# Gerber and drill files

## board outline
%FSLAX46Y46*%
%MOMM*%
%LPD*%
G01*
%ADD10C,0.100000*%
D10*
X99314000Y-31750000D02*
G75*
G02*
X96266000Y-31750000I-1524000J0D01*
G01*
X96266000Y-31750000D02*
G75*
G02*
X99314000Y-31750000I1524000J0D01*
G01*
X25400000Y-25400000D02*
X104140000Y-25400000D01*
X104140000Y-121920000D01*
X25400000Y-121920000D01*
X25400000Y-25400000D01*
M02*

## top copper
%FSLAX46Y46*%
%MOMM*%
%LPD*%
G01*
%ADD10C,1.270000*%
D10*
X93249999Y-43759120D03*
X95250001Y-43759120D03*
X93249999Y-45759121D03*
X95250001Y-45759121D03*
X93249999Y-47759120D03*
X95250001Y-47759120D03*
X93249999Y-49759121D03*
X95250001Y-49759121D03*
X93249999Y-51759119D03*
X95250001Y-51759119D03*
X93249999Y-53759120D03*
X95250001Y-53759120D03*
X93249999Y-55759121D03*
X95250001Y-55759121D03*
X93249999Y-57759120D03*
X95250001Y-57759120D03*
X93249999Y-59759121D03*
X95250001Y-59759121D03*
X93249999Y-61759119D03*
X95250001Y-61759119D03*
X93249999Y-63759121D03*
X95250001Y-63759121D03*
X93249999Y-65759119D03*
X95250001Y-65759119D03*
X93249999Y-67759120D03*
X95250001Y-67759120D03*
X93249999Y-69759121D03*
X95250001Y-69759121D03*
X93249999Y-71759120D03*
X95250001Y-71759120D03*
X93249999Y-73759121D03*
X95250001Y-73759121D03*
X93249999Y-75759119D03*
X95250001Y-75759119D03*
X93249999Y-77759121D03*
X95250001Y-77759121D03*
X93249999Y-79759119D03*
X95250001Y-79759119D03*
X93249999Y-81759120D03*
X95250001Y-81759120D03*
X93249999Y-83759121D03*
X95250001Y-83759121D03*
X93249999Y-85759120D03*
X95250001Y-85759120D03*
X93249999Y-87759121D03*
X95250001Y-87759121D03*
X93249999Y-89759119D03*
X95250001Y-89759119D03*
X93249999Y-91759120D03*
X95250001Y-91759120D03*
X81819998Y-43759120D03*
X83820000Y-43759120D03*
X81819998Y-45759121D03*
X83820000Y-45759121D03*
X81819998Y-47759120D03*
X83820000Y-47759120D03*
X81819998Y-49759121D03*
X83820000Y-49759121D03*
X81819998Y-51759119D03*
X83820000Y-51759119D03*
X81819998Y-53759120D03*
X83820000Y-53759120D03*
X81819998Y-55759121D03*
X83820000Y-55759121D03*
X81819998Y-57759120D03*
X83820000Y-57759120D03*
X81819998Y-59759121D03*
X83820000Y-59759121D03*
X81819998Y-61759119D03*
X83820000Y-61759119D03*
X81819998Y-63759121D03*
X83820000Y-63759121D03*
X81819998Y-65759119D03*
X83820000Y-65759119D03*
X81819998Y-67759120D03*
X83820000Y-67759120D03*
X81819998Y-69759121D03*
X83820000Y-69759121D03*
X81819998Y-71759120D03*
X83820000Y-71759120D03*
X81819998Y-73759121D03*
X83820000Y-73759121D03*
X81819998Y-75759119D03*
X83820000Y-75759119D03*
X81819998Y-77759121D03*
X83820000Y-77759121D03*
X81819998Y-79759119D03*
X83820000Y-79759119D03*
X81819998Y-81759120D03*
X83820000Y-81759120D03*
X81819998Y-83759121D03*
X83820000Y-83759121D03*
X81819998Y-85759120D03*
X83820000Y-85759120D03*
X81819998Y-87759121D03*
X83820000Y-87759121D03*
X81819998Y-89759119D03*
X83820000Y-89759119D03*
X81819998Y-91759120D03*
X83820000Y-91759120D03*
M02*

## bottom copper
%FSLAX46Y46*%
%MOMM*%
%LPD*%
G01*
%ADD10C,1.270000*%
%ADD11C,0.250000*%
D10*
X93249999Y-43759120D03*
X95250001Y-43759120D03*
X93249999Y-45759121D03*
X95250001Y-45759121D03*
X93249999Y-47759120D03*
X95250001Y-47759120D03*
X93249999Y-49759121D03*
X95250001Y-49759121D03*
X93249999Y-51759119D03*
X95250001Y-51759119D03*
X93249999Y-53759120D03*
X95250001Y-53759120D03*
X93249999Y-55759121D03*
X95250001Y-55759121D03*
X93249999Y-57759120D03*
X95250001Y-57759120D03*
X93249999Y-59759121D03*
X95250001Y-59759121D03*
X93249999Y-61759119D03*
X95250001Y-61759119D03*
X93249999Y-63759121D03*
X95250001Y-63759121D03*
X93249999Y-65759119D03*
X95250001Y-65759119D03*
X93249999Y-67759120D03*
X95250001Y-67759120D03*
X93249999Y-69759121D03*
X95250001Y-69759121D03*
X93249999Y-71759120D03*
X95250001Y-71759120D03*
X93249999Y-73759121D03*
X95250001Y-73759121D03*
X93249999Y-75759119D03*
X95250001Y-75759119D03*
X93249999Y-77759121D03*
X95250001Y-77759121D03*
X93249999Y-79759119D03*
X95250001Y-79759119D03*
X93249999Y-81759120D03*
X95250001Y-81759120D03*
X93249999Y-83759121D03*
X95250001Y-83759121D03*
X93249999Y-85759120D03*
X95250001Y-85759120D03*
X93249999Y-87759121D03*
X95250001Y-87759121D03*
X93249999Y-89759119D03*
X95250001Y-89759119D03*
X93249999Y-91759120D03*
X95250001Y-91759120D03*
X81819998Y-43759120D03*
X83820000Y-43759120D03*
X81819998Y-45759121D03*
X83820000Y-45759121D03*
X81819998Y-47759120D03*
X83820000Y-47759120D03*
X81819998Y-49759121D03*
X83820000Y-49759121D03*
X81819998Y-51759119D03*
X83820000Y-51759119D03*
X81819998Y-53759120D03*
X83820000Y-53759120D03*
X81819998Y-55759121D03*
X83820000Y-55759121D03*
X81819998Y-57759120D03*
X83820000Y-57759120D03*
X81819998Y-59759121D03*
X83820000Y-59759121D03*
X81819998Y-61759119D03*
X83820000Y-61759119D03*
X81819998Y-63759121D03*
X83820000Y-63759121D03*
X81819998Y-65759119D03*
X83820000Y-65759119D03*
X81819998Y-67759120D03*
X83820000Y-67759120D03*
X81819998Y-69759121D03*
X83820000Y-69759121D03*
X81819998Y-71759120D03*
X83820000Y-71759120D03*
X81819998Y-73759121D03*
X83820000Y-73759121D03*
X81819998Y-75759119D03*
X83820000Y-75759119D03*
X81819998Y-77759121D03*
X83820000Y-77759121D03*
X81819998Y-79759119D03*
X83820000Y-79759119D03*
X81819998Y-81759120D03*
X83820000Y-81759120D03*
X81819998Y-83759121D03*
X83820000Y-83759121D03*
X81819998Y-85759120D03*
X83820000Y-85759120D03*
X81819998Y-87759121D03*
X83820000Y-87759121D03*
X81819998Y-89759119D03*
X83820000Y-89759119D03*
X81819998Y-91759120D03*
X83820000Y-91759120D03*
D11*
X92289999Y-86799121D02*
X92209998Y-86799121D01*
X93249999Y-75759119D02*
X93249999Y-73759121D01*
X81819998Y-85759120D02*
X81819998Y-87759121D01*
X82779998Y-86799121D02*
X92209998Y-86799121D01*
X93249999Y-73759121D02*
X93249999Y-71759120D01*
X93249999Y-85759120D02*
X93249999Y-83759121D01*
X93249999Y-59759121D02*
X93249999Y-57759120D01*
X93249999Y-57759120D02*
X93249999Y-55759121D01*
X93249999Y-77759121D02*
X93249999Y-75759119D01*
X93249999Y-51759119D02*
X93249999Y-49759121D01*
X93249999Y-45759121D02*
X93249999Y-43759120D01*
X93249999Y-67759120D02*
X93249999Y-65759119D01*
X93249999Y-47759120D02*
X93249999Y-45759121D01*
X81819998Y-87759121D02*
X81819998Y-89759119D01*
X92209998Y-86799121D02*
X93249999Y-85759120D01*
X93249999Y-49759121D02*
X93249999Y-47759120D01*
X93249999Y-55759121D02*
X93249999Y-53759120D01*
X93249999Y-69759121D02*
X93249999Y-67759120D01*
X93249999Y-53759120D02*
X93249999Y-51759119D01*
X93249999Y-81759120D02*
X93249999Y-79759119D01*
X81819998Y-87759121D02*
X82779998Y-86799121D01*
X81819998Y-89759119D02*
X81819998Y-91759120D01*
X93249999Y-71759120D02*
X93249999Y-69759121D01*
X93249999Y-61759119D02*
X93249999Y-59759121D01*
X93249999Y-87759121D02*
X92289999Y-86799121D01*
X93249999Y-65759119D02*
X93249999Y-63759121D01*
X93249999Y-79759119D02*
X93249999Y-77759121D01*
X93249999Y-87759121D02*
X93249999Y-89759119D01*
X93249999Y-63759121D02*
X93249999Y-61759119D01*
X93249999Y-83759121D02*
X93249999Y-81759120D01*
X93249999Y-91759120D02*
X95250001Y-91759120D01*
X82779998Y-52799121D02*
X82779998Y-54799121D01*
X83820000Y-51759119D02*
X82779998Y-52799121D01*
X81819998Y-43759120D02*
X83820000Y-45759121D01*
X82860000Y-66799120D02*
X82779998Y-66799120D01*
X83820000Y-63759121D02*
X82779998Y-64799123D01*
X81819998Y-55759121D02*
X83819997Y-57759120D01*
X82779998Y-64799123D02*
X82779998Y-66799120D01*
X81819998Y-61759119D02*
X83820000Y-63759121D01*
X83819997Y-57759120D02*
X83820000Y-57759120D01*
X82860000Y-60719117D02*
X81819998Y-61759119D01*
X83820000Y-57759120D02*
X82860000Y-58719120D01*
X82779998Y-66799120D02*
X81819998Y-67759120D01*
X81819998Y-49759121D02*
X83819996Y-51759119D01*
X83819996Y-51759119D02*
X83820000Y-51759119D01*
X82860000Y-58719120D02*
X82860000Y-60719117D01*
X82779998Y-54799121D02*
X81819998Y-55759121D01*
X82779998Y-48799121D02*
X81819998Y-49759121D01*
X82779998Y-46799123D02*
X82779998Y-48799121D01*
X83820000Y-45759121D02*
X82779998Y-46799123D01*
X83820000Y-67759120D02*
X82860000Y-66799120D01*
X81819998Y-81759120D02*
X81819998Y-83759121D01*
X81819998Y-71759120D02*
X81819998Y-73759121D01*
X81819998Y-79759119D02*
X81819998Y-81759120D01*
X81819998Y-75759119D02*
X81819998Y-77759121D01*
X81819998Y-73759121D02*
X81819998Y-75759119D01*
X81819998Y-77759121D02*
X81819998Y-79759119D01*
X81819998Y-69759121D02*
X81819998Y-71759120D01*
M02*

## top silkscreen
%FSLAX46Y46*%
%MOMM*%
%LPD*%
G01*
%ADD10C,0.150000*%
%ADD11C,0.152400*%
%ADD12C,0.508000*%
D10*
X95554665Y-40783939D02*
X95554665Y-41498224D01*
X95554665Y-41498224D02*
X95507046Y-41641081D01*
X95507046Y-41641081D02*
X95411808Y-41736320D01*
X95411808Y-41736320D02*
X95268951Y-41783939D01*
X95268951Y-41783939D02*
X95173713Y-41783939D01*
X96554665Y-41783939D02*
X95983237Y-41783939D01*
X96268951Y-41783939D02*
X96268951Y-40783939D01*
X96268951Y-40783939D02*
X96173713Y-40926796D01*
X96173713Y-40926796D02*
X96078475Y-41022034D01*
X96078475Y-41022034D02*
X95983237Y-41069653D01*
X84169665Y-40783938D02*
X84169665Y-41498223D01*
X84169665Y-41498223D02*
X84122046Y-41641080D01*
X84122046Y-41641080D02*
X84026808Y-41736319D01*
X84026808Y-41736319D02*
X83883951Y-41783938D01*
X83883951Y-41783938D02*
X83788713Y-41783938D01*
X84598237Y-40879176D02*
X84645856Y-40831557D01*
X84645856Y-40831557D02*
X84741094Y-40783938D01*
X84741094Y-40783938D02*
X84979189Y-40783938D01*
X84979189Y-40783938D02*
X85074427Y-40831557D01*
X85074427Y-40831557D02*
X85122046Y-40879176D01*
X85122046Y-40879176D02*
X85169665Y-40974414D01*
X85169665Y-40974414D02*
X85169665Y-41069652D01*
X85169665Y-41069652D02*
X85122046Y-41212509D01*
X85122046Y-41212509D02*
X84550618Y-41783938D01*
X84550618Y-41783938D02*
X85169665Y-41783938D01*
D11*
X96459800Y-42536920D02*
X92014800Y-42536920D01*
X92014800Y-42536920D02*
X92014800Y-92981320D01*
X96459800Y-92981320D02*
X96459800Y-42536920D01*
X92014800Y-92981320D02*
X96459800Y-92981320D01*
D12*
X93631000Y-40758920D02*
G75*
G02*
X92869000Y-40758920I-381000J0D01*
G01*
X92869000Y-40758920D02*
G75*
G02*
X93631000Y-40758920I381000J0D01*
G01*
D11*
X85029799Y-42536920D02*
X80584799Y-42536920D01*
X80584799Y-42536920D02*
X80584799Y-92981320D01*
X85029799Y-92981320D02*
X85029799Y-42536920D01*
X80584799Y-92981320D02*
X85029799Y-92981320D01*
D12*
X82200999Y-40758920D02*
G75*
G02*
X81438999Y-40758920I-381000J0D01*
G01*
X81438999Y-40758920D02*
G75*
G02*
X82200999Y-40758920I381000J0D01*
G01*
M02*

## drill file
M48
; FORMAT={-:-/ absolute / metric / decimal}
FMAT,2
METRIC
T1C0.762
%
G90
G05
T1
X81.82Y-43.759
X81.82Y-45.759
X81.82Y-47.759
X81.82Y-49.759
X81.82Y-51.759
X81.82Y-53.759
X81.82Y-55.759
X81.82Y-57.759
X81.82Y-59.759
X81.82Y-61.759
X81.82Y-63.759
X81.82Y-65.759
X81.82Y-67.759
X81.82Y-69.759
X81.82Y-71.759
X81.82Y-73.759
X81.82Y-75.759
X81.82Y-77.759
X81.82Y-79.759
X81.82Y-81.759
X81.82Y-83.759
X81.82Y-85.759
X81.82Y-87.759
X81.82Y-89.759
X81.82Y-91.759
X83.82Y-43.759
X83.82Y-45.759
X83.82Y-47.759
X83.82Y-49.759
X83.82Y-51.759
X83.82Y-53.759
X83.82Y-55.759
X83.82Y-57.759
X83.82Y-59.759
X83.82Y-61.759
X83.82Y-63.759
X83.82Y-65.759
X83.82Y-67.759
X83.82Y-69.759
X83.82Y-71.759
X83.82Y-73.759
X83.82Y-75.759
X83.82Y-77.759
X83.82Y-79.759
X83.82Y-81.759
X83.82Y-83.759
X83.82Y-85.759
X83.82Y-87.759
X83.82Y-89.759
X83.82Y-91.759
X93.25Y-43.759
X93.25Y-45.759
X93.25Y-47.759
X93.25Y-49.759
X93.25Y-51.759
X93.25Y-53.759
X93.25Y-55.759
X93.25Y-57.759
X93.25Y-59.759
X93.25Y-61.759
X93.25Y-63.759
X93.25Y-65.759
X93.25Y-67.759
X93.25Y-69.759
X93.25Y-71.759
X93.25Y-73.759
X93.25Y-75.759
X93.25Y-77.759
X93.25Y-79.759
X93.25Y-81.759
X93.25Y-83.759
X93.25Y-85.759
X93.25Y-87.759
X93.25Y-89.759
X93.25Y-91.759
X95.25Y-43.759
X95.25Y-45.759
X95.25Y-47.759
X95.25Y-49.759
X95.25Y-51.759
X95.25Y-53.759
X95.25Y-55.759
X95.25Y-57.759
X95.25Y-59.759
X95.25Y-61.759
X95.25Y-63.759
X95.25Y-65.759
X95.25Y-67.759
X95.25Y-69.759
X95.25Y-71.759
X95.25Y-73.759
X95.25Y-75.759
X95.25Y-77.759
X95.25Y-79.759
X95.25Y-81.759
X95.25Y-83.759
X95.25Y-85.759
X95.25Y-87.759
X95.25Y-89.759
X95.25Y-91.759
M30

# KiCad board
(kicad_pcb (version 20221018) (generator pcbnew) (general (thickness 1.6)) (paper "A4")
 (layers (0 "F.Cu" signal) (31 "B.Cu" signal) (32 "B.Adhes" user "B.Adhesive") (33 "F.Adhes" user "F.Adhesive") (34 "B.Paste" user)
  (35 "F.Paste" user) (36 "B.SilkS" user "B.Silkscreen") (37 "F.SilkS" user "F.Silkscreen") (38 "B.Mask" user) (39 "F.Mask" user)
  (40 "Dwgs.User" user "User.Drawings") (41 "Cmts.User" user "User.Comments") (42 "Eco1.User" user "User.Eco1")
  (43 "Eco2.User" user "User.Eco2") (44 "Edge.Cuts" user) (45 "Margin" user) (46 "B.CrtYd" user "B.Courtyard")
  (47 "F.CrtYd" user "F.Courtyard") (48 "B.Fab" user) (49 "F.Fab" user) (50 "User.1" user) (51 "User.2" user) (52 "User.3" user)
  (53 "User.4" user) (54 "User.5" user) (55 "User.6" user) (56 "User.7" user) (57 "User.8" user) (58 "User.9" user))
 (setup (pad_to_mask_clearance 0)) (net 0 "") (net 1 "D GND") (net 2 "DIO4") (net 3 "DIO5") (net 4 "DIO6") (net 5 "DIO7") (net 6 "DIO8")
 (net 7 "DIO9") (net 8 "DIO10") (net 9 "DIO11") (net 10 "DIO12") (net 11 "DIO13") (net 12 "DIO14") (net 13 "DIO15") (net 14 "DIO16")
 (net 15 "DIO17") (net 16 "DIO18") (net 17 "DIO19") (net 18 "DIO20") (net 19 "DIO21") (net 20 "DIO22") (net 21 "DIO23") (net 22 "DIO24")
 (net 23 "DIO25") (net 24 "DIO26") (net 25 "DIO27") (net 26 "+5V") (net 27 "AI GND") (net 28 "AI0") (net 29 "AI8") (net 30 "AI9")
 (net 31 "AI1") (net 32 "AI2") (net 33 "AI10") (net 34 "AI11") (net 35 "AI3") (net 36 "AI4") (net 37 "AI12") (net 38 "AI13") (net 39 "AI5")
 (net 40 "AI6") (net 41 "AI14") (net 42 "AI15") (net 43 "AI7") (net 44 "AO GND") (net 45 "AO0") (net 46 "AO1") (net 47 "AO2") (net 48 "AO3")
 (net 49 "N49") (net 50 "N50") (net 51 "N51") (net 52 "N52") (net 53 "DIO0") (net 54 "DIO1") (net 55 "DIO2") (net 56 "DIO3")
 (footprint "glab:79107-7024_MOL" (layer "F.Cu") (at 93.25 43.75912 -90)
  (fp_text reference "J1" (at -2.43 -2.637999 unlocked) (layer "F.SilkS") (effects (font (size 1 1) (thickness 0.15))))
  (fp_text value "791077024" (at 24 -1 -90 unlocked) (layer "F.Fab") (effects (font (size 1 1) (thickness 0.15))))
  (fp_line (start -1.2222 -3.2098) (end -1.2222 1.2352) (stroke (width 0.1524) (type solid)) (layer "F.SilkS"))
  (fp_line (start -1.2222 1.2352) (end 49.2222 1.2352) (stroke (width 0.1524) (type solid)) (layer "F.SilkS"))
  (fp_line (start 49.2222 -3.2098) (end -1.2222 -3.2098) (stroke (width 0.1524) (type solid)) (layer "F.SilkS"))
  (fp_line (start 49.2222 1.2352) (end 49.2222 -3.2098) (stroke (width 0.1524) (type solid)) (layer "F.SilkS"))
  (fp_circle (center -3.0002 0) (end -2.6192 0) (stroke (width 0.508) (type solid)) (fill none) (layer "F.SilkS"))
  (pad "1" thru_hole circle (at 0 0.000001 270) (size 1.27 1.27) (drill 0.762) (layers "*.Cu" "*.Mask") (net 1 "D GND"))
  (pad "2" thru_hole circle (at 0 -2.000001 270) (size 1.27 1.27) (drill 0.762) (layers "*.Cu" "*.Mask") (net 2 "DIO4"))
  (pad "3" thru_hole circle (at 2.000001 0.000001 270) (size 1.27 1.27) (drill 0.762) (layers "*.Cu" "*.Mask") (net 1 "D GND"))
  (pad "4" thru_hole circle (at 2.000001 -2.000001 270) (size 1.27 1.27) (drill 0.762) (layers "*.Cu" "*.Mask") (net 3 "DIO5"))
  (pad "5" thru_hole circle (at 4 0.000001 270) (size 1.27 1.27) (drill 0.762) (layers "*.Cu" "*.Mask") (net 1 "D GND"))
  (pad "6" thru_hole circle (at 4 -2.000001 270) (size 1.27 1.27) (drill 0.762) (layers "*.Cu" "*.Mask") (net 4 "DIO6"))
  (pad "7" thru_hole circle (at 6.000001 0.000001 270) (size 1.27 1.27) (drill 0.762) (layers "*.Cu" "*.Mask") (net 1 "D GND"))
  (pad "8" thru_hole circle (at 6.000001 -2.000001 270) (size 1.27 1.27) (drill 0.762) (layers "*.Cu" "*.Mask") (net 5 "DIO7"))
  (pad "9" thru_hole circle (at 7.999999 0.000001 270) (size 1.27 1.27) (drill 0.762) (layers "*.Cu" "*.Mask") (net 1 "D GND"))
  (pad "10" thru_hole circle (at 7.999999 -2.000001 270) (size 1.27 1.27) (drill 0.762) (layers "*.Cu" "*.Mask") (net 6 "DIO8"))
  (pad "11" thru_hole circle (at 10 0.000001 270) (size 1.27 1.27) (drill 0.762) (layers "*.Cu" "*.Mask") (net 1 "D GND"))
  (pad "12" thru_hole circle (at 10 -2.000001 270) (size 1.27 1.27) (drill 0.762) (layers "*.Cu" "*.Mask") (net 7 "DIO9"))
  (pad "13" thru_hole circle (at 12.000001 0.000001 270) (size 1.27 1.27) (drill 0.762) (layers "*.Cu" "*.Mask") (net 1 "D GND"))
  (pad "14" thru_hole circle (at 12.000001 -2.000001 270) (size 1.27 1.27) (drill 0.762) (layers "*.Cu" "*.Mask") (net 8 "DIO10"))
  (pad "15" thru_hole circle (at 14 0.000001 270) (size 1.27 1.27) (drill 0.762) (layers "*.Cu" "*.Mask") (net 1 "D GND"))
  (pad "16" thru_hole circle (at 14 -2.000001 270) (size 1.27 1.27) (drill 0.762) (layers "*.Cu" "*.Mask") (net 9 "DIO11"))
  (pad "17" thru_hole circle (at 16.000001 0.000001 270) (size 1.27 1.27) (drill 0.762) (layers "*.Cu" "*.Mask") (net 1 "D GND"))
  (pad "18" thru_hole circle (at 16.000001 -2.000001 270) (size 1.27 1.27) (drill 0.762) (layers "*.Cu" "*.Mask") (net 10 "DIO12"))
  (pad "19" thru_hole circle (at 17.999999 0.000001 270) (size 1.27 1.27) (drill 0.762) (layers "*.Cu" "*.Mask") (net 1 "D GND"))
  (pad "20" thru_hole circle (at 17.999999 -2.000001 270) (size 1.27 1.27) (drill 0.762) (layers "*.Cu" "*.Mask") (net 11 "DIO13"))
  (pad "21" thru_hole circle (at 20.000001 0.000001 270) (size 1.27 1.27) (drill 0.762) (layers "*.Cu" "*.Mask") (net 1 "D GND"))
  (pad "22" thru_hole circle (at 20.000001 -2.000001 270) (size 1.27 1.27) (drill 0.762) (layers "*.Cu" "*.Mask") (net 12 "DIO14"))
  (pad "23" thru_hole circle (at 21.999999 0.000001 270) (size 1.27 1.27) (drill 0.762) (layers "*.Cu" "*.Mask") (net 1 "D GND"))
  (pad "24" thru_hole circle (at 21.999999 -2.000001 270) (size 1.27 1.27) (drill 0.762) (layers "*.Cu" "*.Mask") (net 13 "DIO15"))
  (pad "25" thru_hole circle (at 24 0.000001 270) (size 1.27 1.27) (drill 0.762) (layers "*.Cu" "*.Mask") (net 1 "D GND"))
  (pad "26" thru_hole circle (at 24 -2.000001 270) (size 1.27 1.27) (drill 0.762) (layers "*.Cu" "*.Mask") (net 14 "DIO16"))
  (pad "27" thru_hole circle (at 26.000001 0.000001 270) (size 1.27 1.27) (drill 0.762) (layers "*.Cu" "*.Mask") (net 1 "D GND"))
  (pad "28" thru_hole circle (at 26.000001 -2.000001 270) (size 1.27 1.27) (drill 0.762) (layers "*.Cu" "*.Mask") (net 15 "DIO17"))
  (pad "29" thru_hole circle (at 28 0.000001 270) (size 1.27 1.27) (drill 0.762) (layers "*.Cu" "*.Mask") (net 1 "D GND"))
  (pad "30" thru_hole circle (at 28 -2.000001 270) (size 1.27 1.27) (drill 0.762) (layers "*.Cu" "*.Mask") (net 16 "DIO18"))
  (pad "31" thru_hole circle (at 30.000001 0.000001 270) (size 1.27 1.27) (drill 0.762) (layers "*.Cu" "*.Mask") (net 1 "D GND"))
  (pad "32" thru_hole circle (at 30.000001 -2.000001 270) (size 1.27 1.27) (drill 0.762) (layers "*.Cu" "*.Mask") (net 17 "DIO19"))
  (pad "33" thru_hole circle (at 31.999999 0.000001 270) (size 1.27 1.27) (drill 0.762) (layers "*.Cu" "*.Mask") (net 1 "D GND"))
  (pad "34" thru_hole circle (at 31.999999 -2.000001 270) (size 1.27 1.27) (drill 0.762) (layers "*.Cu" "*.Mask") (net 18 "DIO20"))
  (pad "35" thru_hole circle (at 34.000001 0.000001 270) (size 1.27 1.27) (drill 0.762) (layers "*.Cu" "*.Mask") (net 1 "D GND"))
  (pad "36" thru_hole circle (at 34.000001 -2.000001 270) (size 1.27 1.27) (drill 0.762) (layers "*.Cu" "*.Mask") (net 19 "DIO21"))
  (pad "37" thru_hole circle (at 35.999999 0.000001 270) (size 1.27 1.27) (drill 0.762) (layers "*.Cu" "*.Mask") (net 1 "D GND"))
  (pad "38" thru_hole circle (at 35.999999 -2.000001 270) (size 1.27 1.27) (drill 0.762) (layers "*.Cu" "*.Mask") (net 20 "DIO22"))
  (pad "39" thru_hole circle (at 38 0.000001 270) (size 1.27 1.27) (drill 0.762) (layers "*.Cu" "*.Mask") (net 1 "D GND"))
  (pad "40" thru_hole circle (at 38 -2.000001 270) (size 1.27 1.27) (drill 0.762) (layers "*.Cu" "*.Mask") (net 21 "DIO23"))
  (pad "41" thru_hole circle (at 40.000001 0.000001 270) (size 1.27 1.27) (drill 0.762) (layers "*.Cu" "*.Mask") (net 1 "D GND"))
  (pad "42" thru_hole circle (at 40.000001 -2.000001 270) (size 1.27 1.27) (drill 0.762) (layers "*.Cu" "*.Mask") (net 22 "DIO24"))
  (pad "43" thru_hole circle (at 42 0.000001 270) (size 1.27 1.27) (drill 0.762) (layers "*.Cu" "*.Mask") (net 1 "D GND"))
  (pad "44" thru_hole circle (at 42 -2.000001 270) (size 1.27 1.27) (drill 0.762) (layers "*.Cu" "*.Mask") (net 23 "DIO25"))
  (pad "45" thru_hole circle (at 44.000001 0.000001 270) (size 1.27 1.27) (drill 0.762) (layers "*.Cu" "*.Mask") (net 1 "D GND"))
  (pad "46" thru_hole circle (at 44.000001 -2.000001 270) (size 1.27 1.27) (drill 0.762) (layers "*.Cu" "*.Mask") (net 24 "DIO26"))
  (pad "47" thru_hole circle (at 45.999999 0.000001 270) (size 1.27 1.27) (drill 0.762) (layers "*.Cu" "*.Mask") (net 1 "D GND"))
  (pad "48" thru_hole circle (at 45.999999 -2.000001 270) (size 1.27 1.27) (drill 0.762) (layers "*.Cu" "*.Mask") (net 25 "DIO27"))
  (pad "49" thru_hole circle (at 48 0.000001 270) (size 1.27 1.27) (drill 0.762) (layers "*.Cu" "*.Mask") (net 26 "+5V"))
  (pad "50" thru_hole circle (at 48 -2.000001 270) (size 1.27 1.27) (drill 0.762) (layers "*.Cu" "*.Mask") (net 26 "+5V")))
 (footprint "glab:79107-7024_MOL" (layer "F.Cu") (at 81.819999 43.75912 -90)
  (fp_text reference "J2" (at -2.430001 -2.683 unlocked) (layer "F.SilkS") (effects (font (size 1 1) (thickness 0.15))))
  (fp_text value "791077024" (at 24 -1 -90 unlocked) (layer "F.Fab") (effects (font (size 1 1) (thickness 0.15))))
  (fp_line (start -1.2222 -3.2098) (end -1.2222 1.2352) (stroke (width 0.1524) (type solid)) (layer "F.SilkS"))
  (fp_line (start -1.2222 1.2352) (end 49.2222 1.2352) (stroke (width 0.1524) (type solid)) (layer "F.SilkS"))
  (fp_line (start 49.2222 -3.2098) (end -1.2222 -3.2098) (stroke (width 0.1524) (type solid)) (layer "F.SilkS"))
  (fp_line (start 49.2222 1.2352) (end 49.2222 -3.2098) (stroke (width 0.1524) (type solid)) (layer "F.SilkS"))
  (fp_circle (center -3.0002 0) (end -2.6192 0) (stroke (width 0.508) (type solid)) (fill none) (layer "F.SilkS"))
  (pad "1" thru_hole circle (at 0 0.000001 270) (size 1.27 1.27) (drill 0.762) (layers "*.Cu" "*.Mask") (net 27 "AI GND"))
  (pad "2" thru_hole circle (at 0 -2.000001 270) (size 1.27 1.27) (drill 0.762) (layers "*.Cu" "*.Mask") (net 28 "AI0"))
  (pad "3" thru_hole circle (at 2.000001 0.000001 270) (size 1.27 1.27) (drill 0.762) (layers "*.Cu" "*.Mask") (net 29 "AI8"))
  (pad "4" thru_hole circle (at 2.000001 -2.000001 270) (size 1.27 1.27) (drill 0.762) (layers "*.Cu" "*.Mask") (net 27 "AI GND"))
  (pad "5" thru_hole circle (at 4 0.000001 270) (size 1.27 1.27) (drill 0.762) (layers "*.Cu" "*.Mask") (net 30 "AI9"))
  (pad "6" thru_hole circle (at 4 -2.000001 270) (size 1.27 1.27) (drill 0.762) (layers "*.Cu" "*.Mask") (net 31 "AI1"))
  (pad "7" thru_hole circle (at 6.000001 0.000001 270) (size 1.27 1.27) (drill 0.762) (layers "*.Cu" "*.Mask") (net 27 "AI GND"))
  (pad "8" thru_hole circle (at 6.000001 -2.000001 270) (size 1.27 1.27) (drill 0.762) (layers "*.Cu" "*.Mask") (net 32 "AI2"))
  (pad "9" thru_hole circle (at 7.999999 0.000001 270) (size 1.27 1.27) (drill 0.762) (layers "*.Cu" "*.Mask") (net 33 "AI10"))
  (pad "10" thru_hole circle (at 7.999999 -2.000001 270) (size 1.27 1.27) (drill 0.762) (layers "*.Cu" "*.Mask") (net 27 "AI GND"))
  (pad "11" thru_hole circle (at 10 0.000001 270) (size 1.27 1.27) (drill 0.762) (layers "*.Cu" "*.Mask") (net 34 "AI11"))
  (pad "12" thru_hole circle (at 10 -2.000001 270) (size 1.27 1.27) (drill 0.762) (layers "*.Cu" "*.Mask") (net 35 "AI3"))
  (pad "13" thru_hole circle (at 12.000001 0.000001 270) (size 1.27 1.27) (drill 0.762) (layers "*.Cu" "*.Mask") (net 27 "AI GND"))
  (pad "14" thru_hole circle (at 12.000001 -2.000001 270) (size 1.27 1.27) (drill 0.762) (layers "*.Cu" "*.Mask") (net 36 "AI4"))
  (pad "15" thru_hole circle (at 14 0.000001 270) (size 1.27 1.27) (drill 0.762) (layers "*.Cu" "*.Mask") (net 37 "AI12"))
  (pad "16" thru_hole circle (at 14 -2.000001 270) (size 1.27 1.27) (drill 0.762) (layers "*.Cu" "*.Mask") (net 27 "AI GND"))
  (pad "17" thru_hole circle (at 16.000001 0.000001 270) (size 1.27 1.27) (drill 0.762) (layers "*.Cu" "*.Mask") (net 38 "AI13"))
  (pad "18" thru_hole circle (at 16.000001 -2.000001 270) (size 1.27 1.27) (drill 0.762) (layers "*.Cu" "*.Mask") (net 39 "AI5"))
  (pad "19" thru_hole circle (at 17.999999 0.000001 270) (size 1.27 1.27) (drill 0.762) (layers "*.Cu" "*.Mask") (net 27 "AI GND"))
  (pad "20" thru_hole circle (at 17.999999 -2.000001 270) (size 1.27 1.27) (drill 0.762) (layers "*.Cu" "*.Mask") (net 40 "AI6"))
  (pad "21" thru_hole circle (at 20.000001 0.000001 270) (size 1.27 1.27) (drill 0.762) (layers "*.Cu" "*.Mask") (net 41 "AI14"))
  (pad "22" thru_hole circle (at 20.000001 -2.000001 270) (size 1.27 1.27) (drill 0.762) (layers "*.Cu" "*.Mask") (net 27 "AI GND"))
  (pad "23" thru_hole circle (at 21.999999 0.000001 270) (size 1.27 1.27) (drill 0.762) (layers "*.Cu" "*.Mask") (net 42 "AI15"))
  (pad "24" thru_hole circle (at 21.999999 -2.000001 270) (size 1.27 1.27) (drill 0.762) (layers "*.Cu" "*.Mask") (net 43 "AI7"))
  (pad "25" thru_hole circle (at 24 0.000001 270) (size 1.27 1.27) (drill 0.762) (layers "*.Cu" "*.Mask") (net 27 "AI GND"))
  (pad "26" thru_hole circle (at 24 -2.000001 270) (size 1.27 1.27) (drill 0.762) (layers "*.Cu" "*.Mask") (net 27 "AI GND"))
  (pad "27" thru_hole circle (at 26.000001 0.000001 270) (size 1.27 1.27) (drill 0.762) (layers "*.Cu" "*.Mask") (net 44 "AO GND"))
  (pad "28" thru_hole circle (at 26.000001 -2.000001 270) (size 1.27 1.27) (drill 0.762) (layers "*.Cu" "*.Mask") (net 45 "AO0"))
  (pad "29" thru_hole circle (at 28 0.000001 270) (size 1.27 1.27) (drill 0.762) (layers "*.Cu" "*.Mask") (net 44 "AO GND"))
  (pad "30" thru_hole circle (at 28 -2.000001 270) (size 1.27 1.27) (drill 0.762) (layers "*.Cu" "*.Mask") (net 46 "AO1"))
  (pad "31" thru_hole circle (at 30.000001 0.000001 270) (size 1.27 1.27) (drill 0.762) (layers "*.Cu" "*.Mask") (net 44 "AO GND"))
  (pad "32" thru_hole circle (at 30.000001 -2.000001 270) (size 1.27 1.27) (drill 0.762) (layers "*.Cu" "*.Mask") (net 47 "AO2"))
  (pad "33" thru_hole circle (at 31.999999 0.000001 270) (size 1.27 1.27) (drill 0.762) (layers "*.Cu" "*.Mask") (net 44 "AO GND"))
  (pad "34" thru_hole circle (at 31.999999 -2.000001 270) (size 1.27 1.27) (drill 0.762) (layers "*.Cu" "*.Mask") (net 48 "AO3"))
  (pad "35" thru_hole circle (at 34.000001 0.000001 270) (size 1.27 1.27) (drill 0.762) (layers "*.Cu" "*.Mask") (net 44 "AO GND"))
  (pad "36" thru_hole circle (at 34.000001 -2.000001 270) (size 1.27 1.27) (drill 0.762) (layers "*.Cu" "*.Mask") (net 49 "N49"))
  (pad "37" thru_hole circle (at 35.999999 0.000001 270) (size 1.27 1.27) (drill 0.762) (layers "*.Cu" "*.Mask") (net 44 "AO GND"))
  (pad "38" thru_hole circle (at 35.999999 -2.000001 270) (size 1.27 1.27) (drill 0.762) (layers "*.Cu" "*.Mask") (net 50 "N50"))
  (pad "39" thru_hole circle (at 38 0.000001 270) (size 1.27 1.27) (drill 0.762) (layers "*.Cu" "*.Mask") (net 44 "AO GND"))
  (pad "40" thru_hole circle (at 38 -2.000001 270) (size 1.27 1.27) (drill 0.762) (layers "*.Cu" "*.Mask") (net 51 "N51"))
  (pad "41" thru_hole circle (at 40.000001 0.000001 270) (size 1.27 1.27) (drill 0.762) (layers "*.Cu" "*.Mask") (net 44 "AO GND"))
  (pad "42" thru_hole circle (at 40.000001 -2.000001 270) (size 1.27 1.27) (drill 0.762) (layers "*.Cu" "*.Mask") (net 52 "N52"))
  (pad "43" thru_hole circle (at 42 0.000001 270) (size 1.27 1.27) (drill 0.762) (layers "*.Cu" "*.Mask") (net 1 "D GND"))
  (pad "44" thru_hole circle (at 42 -2.000001 270) (size 1.27 1.27) (drill 0.762) (layers "*.Cu" "*.Mask") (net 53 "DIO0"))
  (pad "45" thru_hole circle (at 44.000001 0.000001 270) (size 1.27 1.27) (drill 0.762) (layers "*.Cu" "*.Mask") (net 1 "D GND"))
  (pad "46" thru_hole circle (at 44.000001 -2.000001 270) (size 1.27 1.27) (drill 0.762) (layers "*.Cu" "*.Mask") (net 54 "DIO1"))
  (pad "47" thru_hole circle (at 45.999999 0.000001 270) (size 1.27 1.27) (drill 0.762) (layers "*.Cu" "*.Mask") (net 1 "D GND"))
  (pad "48" thru_hole circle (at 45.999999 -2.000001 270) (size 1.27 1.27) (drill 0.762) (layers "*.Cu" "*.Mask") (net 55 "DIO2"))
  (pad "49" thru_hole circle (at 48 0.000001 270) (size 1.27 1.27) (drill 0.762) (layers "*.Cu" "*.Mask") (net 1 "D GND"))
  (pad "50" thru_hole circle (at 48 -2.000001 270) (size 1.27 1.27) (drill 0.762) (layers "*.Cu" "*.Mask") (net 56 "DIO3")))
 (gr_circle (center 97.79 31.75) (end 99.314 31.75) (stroke (width 0.1) (type default)) (fill none) (layer "Edge.Cuts"))
 (gr_rect (start 25.4 25.4) (end 104.14 121.92) (stroke (width 0.1) (type default)) (fill none) (layer "Edge.Cuts"))
 (segment (start 92.289999 86.799121) (end 92.209998 86.799121) (width 0.25) (layer "B.Cu") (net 1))
 (segment (start 93.249999 75.759119) (end 93.249999 73.759121) (width 0.25) (layer "B.Cu") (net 1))
 (segment (start 81.819998 85.75912) (end 81.819998 87.759121) (width 0.25) (layer "B.Cu") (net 1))
 (segment (start 82.779998 86.799121) (end 92.209998 86.799121) (width 0.25) (layer "B.Cu") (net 1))
 (segment (start 93.249999 73.759121) (end 93.249999 71.75912) (width 0.25) (layer "B.Cu") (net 1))
 (segment (start 93.249999 85.75912) (end 93.249999 83.759121) (width 0.25) (layer "B.Cu") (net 1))
 (segment (start 93.249999 59.759121) (end 93.249999 57.75912) (width 0.25) (layer "B.Cu") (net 1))
 (segment (start 93.249999 57.75912) (end 93.249999 55.759121) (width 0.25) (layer "B.Cu") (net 1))
 (segment (start 93.249999 77.759121) (end 93.249999 75.759119) (width 0.25) (layer "B.Cu") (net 1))
 (segment (start 93.249999 51.759119) (end 93.249999 49.759121) (width 0.25) (layer "B.Cu") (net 1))
 (segment (start 93.249999 45.759121) (end 93.249999 43.75912) (width 0.25) (layer "B.Cu") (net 1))
 (segment (start 93.249999 67.75912) (end 93.249999 65.759119) (width 0.25) (layer "B.Cu") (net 1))
 (segment (start 93.249999 47.75912) (end 93.249999 45.759121) (width 0.25) (layer "B.Cu") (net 1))
 (segment (start 81.819998 87.759121) (end 81.819998 89.759119) (width 0.25) (layer "B.Cu") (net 1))
 (segment (start 92.209998 86.799121) (end 93.249999 85.75912) (width 0.25) (layer "B.Cu") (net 1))
 (segment (start 93.249999 49.759121) (end 93.249999 47.75912) (width 0.25) (layer "B.Cu") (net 1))
 (segment (start 93.249999 55.759121) (end 93.249999 53.75912) (width 0.25) (layer "B.Cu") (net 1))
 (segment (start 93.249999 69.759121) (end 93.249999 67.75912) (width 0.25) (layer "B.Cu") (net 1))
 (segment (start 93.249999 53.75912) (end 93.249999 51.759119) (width 0.25) (layer "B.Cu") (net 1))
 (segment (start 93.249999 81.75912) (end 93.249999 79.759119) (width 0.25) (layer "B.Cu") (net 1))
 (segment (start 81.819998 87.759121) (end 82.779998 86.799121) (width 0.25) (layer "B.Cu") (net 1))
 (segment (start 81.819998 89.759119) (end 81.819998 91.75912) (width 0.25) (layer "B.Cu") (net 1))
 (segment (start 93.249999 71.75912) (end 93.249999 69.759121) (width 0.25) (layer "B.Cu") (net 1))
 (segment (start 93.249999 61.759119) (end 93.249999 59.759121) (width 0.25) (layer "B.Cu") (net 1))
 (segment (start 93.249999 87.759121) (end 92.289999 86.799121) (width 0.25) (layer "B.Cu") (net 1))
 (segment (start 93.249999 65.759119) (end 93.249999 63.759121) (width 0.25) (layer "B.Cu") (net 1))
 (segment (start 93.249999 79.759119) (end 93.249999 77.759121) (width 0.25) (layer "B.Cu") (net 1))
 (segment (start 93.249999 87.759121) (end 93.249999 89.759119) (width 0.25) (layer "B.Cu") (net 1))
 (segment (start 93.249999 63.759121) (end 93.249999 61.759119) (width 0.25) (layer "B.Cu") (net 1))
 (segment (start 93.249999 83.759121) (end 93.249999 81.75912) (width 0.25) (layer "B.Cu") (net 1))
 (segment (start 93.249999 91.75912) (end 95.250001 91.75912) (width 0.25) (layer "B.Cu") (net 26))
 (segment (start 82.779998 52.799121) (end 82.779998 54.799121) (width 0.25) (layer "B.Cu") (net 27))
 (segment (start 83.82 51.759119) (end 82.779998 52.799121) (width 0.25) (layer "B.Cu") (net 27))
 (segment (start 81.819998 43.75912) (end 83.82 45.759121) (width 0.25) (layer "B.Cu") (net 27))
 (segment (start 82.86 66.79912) (end 82.779998 66.79912) (width 0.25) (layer "B.Cu") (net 27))
 (segment (start 83.82 63.759121) (end 82.779998 64.799123) (width 0.25) (layer "B.Cu") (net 27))
 (segment (start 81.819998 55.759121) (end 83.819997 57.75912) (width 0.25) (layer "B.Cu") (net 27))
 (segment (start 82.779998 64.799123) (end 82.779998 66.79912) (width 0.25) (layer "B.Cu") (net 27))
 (segment (start 81.819998 61.759119) (end 83.82 63.759121) (width 0.25) (layer "B.Cu") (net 27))
 (segment (start 83.819997 57.75912) (end 83.82 57.75912) (width 0.25) (layer "B.Cu") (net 27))
 (segment (start 82.86 60.719117) (end 81.819998 61.759119) (width 0.25) (layer "B.Cu") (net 27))
 (segment (start 83.82 57.75912) (end 82.86 58.71912) (width 0.25) (layer "B.Cu") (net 27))
 (segment (start 82.779998 66.79912) (end 81.819998 67.75912) (width 0.25) (layer "B.Cu") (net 27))
 (segment (start 81.819998 49.759121) (end 83.819996 51.759119) (width 0.25) (layer "B.Cu") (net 27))
 (segment (start 83.819996 51.759119) (end 83.82 51.759119) (width 0.25) (layer "B.Cu") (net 27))
 (segment (start 82.86 58.71912) (end 82.86 60.719117) (width 0.25) (layer "B.Cu") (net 27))
 (segment (start 82.779998 54.799121) (end 81.819998 55.759121) (width 0.25) (layer "B.Cu") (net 27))
 (segment (start 82.779998 48.799121) (end 81.819998 49.759121) (width 0.25) (layer "B.Cu") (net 27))
 (segment (start 82.779998 46.799123) (end 82.779998 48.799121) (width 0.25) (layer "B.Cu") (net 27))
 (segment (start 83.82 45.759121) (end 82.779998 46.799123) (width 0.25) (layer "B.Cu") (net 27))
 (segment (start 83.82 67.75912) (end 82.86 66.79912) (width 0.25) (layer "B.Cu") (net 27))
 (segment (start 81.819998 81.75912) (end 81.819998 83.759121) (width 0.25) (layer "B.Cu") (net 44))
 (segment (start 81.819998 71.75912) (end 81.819998 73.759121) (width 0.25) (layer "B.Cu") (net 44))
 (segment (start 81.819998 79.759119) (end 81.819998 81.75912) (width 0.25) (layer "B.Cu") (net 44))
 (segment (start 81.819998 75.759119) (end 81.819998 77.759121) (width 0.25) (layer "B.Cu") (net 44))
 (segment (start 81.819998 73.759121) (end 81.819998 75.759119) (width 0.25) (layer "B.Cu") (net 44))
 (segment (start 81.819998 77.759121) (end 81.819998 79.759119) (width 0.25) (layer "B.Cu") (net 44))
 (segment (start 81.819998 69.759121) (end 81.819998 71.75912) (width 0.25) (layer "B.Cu") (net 44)))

